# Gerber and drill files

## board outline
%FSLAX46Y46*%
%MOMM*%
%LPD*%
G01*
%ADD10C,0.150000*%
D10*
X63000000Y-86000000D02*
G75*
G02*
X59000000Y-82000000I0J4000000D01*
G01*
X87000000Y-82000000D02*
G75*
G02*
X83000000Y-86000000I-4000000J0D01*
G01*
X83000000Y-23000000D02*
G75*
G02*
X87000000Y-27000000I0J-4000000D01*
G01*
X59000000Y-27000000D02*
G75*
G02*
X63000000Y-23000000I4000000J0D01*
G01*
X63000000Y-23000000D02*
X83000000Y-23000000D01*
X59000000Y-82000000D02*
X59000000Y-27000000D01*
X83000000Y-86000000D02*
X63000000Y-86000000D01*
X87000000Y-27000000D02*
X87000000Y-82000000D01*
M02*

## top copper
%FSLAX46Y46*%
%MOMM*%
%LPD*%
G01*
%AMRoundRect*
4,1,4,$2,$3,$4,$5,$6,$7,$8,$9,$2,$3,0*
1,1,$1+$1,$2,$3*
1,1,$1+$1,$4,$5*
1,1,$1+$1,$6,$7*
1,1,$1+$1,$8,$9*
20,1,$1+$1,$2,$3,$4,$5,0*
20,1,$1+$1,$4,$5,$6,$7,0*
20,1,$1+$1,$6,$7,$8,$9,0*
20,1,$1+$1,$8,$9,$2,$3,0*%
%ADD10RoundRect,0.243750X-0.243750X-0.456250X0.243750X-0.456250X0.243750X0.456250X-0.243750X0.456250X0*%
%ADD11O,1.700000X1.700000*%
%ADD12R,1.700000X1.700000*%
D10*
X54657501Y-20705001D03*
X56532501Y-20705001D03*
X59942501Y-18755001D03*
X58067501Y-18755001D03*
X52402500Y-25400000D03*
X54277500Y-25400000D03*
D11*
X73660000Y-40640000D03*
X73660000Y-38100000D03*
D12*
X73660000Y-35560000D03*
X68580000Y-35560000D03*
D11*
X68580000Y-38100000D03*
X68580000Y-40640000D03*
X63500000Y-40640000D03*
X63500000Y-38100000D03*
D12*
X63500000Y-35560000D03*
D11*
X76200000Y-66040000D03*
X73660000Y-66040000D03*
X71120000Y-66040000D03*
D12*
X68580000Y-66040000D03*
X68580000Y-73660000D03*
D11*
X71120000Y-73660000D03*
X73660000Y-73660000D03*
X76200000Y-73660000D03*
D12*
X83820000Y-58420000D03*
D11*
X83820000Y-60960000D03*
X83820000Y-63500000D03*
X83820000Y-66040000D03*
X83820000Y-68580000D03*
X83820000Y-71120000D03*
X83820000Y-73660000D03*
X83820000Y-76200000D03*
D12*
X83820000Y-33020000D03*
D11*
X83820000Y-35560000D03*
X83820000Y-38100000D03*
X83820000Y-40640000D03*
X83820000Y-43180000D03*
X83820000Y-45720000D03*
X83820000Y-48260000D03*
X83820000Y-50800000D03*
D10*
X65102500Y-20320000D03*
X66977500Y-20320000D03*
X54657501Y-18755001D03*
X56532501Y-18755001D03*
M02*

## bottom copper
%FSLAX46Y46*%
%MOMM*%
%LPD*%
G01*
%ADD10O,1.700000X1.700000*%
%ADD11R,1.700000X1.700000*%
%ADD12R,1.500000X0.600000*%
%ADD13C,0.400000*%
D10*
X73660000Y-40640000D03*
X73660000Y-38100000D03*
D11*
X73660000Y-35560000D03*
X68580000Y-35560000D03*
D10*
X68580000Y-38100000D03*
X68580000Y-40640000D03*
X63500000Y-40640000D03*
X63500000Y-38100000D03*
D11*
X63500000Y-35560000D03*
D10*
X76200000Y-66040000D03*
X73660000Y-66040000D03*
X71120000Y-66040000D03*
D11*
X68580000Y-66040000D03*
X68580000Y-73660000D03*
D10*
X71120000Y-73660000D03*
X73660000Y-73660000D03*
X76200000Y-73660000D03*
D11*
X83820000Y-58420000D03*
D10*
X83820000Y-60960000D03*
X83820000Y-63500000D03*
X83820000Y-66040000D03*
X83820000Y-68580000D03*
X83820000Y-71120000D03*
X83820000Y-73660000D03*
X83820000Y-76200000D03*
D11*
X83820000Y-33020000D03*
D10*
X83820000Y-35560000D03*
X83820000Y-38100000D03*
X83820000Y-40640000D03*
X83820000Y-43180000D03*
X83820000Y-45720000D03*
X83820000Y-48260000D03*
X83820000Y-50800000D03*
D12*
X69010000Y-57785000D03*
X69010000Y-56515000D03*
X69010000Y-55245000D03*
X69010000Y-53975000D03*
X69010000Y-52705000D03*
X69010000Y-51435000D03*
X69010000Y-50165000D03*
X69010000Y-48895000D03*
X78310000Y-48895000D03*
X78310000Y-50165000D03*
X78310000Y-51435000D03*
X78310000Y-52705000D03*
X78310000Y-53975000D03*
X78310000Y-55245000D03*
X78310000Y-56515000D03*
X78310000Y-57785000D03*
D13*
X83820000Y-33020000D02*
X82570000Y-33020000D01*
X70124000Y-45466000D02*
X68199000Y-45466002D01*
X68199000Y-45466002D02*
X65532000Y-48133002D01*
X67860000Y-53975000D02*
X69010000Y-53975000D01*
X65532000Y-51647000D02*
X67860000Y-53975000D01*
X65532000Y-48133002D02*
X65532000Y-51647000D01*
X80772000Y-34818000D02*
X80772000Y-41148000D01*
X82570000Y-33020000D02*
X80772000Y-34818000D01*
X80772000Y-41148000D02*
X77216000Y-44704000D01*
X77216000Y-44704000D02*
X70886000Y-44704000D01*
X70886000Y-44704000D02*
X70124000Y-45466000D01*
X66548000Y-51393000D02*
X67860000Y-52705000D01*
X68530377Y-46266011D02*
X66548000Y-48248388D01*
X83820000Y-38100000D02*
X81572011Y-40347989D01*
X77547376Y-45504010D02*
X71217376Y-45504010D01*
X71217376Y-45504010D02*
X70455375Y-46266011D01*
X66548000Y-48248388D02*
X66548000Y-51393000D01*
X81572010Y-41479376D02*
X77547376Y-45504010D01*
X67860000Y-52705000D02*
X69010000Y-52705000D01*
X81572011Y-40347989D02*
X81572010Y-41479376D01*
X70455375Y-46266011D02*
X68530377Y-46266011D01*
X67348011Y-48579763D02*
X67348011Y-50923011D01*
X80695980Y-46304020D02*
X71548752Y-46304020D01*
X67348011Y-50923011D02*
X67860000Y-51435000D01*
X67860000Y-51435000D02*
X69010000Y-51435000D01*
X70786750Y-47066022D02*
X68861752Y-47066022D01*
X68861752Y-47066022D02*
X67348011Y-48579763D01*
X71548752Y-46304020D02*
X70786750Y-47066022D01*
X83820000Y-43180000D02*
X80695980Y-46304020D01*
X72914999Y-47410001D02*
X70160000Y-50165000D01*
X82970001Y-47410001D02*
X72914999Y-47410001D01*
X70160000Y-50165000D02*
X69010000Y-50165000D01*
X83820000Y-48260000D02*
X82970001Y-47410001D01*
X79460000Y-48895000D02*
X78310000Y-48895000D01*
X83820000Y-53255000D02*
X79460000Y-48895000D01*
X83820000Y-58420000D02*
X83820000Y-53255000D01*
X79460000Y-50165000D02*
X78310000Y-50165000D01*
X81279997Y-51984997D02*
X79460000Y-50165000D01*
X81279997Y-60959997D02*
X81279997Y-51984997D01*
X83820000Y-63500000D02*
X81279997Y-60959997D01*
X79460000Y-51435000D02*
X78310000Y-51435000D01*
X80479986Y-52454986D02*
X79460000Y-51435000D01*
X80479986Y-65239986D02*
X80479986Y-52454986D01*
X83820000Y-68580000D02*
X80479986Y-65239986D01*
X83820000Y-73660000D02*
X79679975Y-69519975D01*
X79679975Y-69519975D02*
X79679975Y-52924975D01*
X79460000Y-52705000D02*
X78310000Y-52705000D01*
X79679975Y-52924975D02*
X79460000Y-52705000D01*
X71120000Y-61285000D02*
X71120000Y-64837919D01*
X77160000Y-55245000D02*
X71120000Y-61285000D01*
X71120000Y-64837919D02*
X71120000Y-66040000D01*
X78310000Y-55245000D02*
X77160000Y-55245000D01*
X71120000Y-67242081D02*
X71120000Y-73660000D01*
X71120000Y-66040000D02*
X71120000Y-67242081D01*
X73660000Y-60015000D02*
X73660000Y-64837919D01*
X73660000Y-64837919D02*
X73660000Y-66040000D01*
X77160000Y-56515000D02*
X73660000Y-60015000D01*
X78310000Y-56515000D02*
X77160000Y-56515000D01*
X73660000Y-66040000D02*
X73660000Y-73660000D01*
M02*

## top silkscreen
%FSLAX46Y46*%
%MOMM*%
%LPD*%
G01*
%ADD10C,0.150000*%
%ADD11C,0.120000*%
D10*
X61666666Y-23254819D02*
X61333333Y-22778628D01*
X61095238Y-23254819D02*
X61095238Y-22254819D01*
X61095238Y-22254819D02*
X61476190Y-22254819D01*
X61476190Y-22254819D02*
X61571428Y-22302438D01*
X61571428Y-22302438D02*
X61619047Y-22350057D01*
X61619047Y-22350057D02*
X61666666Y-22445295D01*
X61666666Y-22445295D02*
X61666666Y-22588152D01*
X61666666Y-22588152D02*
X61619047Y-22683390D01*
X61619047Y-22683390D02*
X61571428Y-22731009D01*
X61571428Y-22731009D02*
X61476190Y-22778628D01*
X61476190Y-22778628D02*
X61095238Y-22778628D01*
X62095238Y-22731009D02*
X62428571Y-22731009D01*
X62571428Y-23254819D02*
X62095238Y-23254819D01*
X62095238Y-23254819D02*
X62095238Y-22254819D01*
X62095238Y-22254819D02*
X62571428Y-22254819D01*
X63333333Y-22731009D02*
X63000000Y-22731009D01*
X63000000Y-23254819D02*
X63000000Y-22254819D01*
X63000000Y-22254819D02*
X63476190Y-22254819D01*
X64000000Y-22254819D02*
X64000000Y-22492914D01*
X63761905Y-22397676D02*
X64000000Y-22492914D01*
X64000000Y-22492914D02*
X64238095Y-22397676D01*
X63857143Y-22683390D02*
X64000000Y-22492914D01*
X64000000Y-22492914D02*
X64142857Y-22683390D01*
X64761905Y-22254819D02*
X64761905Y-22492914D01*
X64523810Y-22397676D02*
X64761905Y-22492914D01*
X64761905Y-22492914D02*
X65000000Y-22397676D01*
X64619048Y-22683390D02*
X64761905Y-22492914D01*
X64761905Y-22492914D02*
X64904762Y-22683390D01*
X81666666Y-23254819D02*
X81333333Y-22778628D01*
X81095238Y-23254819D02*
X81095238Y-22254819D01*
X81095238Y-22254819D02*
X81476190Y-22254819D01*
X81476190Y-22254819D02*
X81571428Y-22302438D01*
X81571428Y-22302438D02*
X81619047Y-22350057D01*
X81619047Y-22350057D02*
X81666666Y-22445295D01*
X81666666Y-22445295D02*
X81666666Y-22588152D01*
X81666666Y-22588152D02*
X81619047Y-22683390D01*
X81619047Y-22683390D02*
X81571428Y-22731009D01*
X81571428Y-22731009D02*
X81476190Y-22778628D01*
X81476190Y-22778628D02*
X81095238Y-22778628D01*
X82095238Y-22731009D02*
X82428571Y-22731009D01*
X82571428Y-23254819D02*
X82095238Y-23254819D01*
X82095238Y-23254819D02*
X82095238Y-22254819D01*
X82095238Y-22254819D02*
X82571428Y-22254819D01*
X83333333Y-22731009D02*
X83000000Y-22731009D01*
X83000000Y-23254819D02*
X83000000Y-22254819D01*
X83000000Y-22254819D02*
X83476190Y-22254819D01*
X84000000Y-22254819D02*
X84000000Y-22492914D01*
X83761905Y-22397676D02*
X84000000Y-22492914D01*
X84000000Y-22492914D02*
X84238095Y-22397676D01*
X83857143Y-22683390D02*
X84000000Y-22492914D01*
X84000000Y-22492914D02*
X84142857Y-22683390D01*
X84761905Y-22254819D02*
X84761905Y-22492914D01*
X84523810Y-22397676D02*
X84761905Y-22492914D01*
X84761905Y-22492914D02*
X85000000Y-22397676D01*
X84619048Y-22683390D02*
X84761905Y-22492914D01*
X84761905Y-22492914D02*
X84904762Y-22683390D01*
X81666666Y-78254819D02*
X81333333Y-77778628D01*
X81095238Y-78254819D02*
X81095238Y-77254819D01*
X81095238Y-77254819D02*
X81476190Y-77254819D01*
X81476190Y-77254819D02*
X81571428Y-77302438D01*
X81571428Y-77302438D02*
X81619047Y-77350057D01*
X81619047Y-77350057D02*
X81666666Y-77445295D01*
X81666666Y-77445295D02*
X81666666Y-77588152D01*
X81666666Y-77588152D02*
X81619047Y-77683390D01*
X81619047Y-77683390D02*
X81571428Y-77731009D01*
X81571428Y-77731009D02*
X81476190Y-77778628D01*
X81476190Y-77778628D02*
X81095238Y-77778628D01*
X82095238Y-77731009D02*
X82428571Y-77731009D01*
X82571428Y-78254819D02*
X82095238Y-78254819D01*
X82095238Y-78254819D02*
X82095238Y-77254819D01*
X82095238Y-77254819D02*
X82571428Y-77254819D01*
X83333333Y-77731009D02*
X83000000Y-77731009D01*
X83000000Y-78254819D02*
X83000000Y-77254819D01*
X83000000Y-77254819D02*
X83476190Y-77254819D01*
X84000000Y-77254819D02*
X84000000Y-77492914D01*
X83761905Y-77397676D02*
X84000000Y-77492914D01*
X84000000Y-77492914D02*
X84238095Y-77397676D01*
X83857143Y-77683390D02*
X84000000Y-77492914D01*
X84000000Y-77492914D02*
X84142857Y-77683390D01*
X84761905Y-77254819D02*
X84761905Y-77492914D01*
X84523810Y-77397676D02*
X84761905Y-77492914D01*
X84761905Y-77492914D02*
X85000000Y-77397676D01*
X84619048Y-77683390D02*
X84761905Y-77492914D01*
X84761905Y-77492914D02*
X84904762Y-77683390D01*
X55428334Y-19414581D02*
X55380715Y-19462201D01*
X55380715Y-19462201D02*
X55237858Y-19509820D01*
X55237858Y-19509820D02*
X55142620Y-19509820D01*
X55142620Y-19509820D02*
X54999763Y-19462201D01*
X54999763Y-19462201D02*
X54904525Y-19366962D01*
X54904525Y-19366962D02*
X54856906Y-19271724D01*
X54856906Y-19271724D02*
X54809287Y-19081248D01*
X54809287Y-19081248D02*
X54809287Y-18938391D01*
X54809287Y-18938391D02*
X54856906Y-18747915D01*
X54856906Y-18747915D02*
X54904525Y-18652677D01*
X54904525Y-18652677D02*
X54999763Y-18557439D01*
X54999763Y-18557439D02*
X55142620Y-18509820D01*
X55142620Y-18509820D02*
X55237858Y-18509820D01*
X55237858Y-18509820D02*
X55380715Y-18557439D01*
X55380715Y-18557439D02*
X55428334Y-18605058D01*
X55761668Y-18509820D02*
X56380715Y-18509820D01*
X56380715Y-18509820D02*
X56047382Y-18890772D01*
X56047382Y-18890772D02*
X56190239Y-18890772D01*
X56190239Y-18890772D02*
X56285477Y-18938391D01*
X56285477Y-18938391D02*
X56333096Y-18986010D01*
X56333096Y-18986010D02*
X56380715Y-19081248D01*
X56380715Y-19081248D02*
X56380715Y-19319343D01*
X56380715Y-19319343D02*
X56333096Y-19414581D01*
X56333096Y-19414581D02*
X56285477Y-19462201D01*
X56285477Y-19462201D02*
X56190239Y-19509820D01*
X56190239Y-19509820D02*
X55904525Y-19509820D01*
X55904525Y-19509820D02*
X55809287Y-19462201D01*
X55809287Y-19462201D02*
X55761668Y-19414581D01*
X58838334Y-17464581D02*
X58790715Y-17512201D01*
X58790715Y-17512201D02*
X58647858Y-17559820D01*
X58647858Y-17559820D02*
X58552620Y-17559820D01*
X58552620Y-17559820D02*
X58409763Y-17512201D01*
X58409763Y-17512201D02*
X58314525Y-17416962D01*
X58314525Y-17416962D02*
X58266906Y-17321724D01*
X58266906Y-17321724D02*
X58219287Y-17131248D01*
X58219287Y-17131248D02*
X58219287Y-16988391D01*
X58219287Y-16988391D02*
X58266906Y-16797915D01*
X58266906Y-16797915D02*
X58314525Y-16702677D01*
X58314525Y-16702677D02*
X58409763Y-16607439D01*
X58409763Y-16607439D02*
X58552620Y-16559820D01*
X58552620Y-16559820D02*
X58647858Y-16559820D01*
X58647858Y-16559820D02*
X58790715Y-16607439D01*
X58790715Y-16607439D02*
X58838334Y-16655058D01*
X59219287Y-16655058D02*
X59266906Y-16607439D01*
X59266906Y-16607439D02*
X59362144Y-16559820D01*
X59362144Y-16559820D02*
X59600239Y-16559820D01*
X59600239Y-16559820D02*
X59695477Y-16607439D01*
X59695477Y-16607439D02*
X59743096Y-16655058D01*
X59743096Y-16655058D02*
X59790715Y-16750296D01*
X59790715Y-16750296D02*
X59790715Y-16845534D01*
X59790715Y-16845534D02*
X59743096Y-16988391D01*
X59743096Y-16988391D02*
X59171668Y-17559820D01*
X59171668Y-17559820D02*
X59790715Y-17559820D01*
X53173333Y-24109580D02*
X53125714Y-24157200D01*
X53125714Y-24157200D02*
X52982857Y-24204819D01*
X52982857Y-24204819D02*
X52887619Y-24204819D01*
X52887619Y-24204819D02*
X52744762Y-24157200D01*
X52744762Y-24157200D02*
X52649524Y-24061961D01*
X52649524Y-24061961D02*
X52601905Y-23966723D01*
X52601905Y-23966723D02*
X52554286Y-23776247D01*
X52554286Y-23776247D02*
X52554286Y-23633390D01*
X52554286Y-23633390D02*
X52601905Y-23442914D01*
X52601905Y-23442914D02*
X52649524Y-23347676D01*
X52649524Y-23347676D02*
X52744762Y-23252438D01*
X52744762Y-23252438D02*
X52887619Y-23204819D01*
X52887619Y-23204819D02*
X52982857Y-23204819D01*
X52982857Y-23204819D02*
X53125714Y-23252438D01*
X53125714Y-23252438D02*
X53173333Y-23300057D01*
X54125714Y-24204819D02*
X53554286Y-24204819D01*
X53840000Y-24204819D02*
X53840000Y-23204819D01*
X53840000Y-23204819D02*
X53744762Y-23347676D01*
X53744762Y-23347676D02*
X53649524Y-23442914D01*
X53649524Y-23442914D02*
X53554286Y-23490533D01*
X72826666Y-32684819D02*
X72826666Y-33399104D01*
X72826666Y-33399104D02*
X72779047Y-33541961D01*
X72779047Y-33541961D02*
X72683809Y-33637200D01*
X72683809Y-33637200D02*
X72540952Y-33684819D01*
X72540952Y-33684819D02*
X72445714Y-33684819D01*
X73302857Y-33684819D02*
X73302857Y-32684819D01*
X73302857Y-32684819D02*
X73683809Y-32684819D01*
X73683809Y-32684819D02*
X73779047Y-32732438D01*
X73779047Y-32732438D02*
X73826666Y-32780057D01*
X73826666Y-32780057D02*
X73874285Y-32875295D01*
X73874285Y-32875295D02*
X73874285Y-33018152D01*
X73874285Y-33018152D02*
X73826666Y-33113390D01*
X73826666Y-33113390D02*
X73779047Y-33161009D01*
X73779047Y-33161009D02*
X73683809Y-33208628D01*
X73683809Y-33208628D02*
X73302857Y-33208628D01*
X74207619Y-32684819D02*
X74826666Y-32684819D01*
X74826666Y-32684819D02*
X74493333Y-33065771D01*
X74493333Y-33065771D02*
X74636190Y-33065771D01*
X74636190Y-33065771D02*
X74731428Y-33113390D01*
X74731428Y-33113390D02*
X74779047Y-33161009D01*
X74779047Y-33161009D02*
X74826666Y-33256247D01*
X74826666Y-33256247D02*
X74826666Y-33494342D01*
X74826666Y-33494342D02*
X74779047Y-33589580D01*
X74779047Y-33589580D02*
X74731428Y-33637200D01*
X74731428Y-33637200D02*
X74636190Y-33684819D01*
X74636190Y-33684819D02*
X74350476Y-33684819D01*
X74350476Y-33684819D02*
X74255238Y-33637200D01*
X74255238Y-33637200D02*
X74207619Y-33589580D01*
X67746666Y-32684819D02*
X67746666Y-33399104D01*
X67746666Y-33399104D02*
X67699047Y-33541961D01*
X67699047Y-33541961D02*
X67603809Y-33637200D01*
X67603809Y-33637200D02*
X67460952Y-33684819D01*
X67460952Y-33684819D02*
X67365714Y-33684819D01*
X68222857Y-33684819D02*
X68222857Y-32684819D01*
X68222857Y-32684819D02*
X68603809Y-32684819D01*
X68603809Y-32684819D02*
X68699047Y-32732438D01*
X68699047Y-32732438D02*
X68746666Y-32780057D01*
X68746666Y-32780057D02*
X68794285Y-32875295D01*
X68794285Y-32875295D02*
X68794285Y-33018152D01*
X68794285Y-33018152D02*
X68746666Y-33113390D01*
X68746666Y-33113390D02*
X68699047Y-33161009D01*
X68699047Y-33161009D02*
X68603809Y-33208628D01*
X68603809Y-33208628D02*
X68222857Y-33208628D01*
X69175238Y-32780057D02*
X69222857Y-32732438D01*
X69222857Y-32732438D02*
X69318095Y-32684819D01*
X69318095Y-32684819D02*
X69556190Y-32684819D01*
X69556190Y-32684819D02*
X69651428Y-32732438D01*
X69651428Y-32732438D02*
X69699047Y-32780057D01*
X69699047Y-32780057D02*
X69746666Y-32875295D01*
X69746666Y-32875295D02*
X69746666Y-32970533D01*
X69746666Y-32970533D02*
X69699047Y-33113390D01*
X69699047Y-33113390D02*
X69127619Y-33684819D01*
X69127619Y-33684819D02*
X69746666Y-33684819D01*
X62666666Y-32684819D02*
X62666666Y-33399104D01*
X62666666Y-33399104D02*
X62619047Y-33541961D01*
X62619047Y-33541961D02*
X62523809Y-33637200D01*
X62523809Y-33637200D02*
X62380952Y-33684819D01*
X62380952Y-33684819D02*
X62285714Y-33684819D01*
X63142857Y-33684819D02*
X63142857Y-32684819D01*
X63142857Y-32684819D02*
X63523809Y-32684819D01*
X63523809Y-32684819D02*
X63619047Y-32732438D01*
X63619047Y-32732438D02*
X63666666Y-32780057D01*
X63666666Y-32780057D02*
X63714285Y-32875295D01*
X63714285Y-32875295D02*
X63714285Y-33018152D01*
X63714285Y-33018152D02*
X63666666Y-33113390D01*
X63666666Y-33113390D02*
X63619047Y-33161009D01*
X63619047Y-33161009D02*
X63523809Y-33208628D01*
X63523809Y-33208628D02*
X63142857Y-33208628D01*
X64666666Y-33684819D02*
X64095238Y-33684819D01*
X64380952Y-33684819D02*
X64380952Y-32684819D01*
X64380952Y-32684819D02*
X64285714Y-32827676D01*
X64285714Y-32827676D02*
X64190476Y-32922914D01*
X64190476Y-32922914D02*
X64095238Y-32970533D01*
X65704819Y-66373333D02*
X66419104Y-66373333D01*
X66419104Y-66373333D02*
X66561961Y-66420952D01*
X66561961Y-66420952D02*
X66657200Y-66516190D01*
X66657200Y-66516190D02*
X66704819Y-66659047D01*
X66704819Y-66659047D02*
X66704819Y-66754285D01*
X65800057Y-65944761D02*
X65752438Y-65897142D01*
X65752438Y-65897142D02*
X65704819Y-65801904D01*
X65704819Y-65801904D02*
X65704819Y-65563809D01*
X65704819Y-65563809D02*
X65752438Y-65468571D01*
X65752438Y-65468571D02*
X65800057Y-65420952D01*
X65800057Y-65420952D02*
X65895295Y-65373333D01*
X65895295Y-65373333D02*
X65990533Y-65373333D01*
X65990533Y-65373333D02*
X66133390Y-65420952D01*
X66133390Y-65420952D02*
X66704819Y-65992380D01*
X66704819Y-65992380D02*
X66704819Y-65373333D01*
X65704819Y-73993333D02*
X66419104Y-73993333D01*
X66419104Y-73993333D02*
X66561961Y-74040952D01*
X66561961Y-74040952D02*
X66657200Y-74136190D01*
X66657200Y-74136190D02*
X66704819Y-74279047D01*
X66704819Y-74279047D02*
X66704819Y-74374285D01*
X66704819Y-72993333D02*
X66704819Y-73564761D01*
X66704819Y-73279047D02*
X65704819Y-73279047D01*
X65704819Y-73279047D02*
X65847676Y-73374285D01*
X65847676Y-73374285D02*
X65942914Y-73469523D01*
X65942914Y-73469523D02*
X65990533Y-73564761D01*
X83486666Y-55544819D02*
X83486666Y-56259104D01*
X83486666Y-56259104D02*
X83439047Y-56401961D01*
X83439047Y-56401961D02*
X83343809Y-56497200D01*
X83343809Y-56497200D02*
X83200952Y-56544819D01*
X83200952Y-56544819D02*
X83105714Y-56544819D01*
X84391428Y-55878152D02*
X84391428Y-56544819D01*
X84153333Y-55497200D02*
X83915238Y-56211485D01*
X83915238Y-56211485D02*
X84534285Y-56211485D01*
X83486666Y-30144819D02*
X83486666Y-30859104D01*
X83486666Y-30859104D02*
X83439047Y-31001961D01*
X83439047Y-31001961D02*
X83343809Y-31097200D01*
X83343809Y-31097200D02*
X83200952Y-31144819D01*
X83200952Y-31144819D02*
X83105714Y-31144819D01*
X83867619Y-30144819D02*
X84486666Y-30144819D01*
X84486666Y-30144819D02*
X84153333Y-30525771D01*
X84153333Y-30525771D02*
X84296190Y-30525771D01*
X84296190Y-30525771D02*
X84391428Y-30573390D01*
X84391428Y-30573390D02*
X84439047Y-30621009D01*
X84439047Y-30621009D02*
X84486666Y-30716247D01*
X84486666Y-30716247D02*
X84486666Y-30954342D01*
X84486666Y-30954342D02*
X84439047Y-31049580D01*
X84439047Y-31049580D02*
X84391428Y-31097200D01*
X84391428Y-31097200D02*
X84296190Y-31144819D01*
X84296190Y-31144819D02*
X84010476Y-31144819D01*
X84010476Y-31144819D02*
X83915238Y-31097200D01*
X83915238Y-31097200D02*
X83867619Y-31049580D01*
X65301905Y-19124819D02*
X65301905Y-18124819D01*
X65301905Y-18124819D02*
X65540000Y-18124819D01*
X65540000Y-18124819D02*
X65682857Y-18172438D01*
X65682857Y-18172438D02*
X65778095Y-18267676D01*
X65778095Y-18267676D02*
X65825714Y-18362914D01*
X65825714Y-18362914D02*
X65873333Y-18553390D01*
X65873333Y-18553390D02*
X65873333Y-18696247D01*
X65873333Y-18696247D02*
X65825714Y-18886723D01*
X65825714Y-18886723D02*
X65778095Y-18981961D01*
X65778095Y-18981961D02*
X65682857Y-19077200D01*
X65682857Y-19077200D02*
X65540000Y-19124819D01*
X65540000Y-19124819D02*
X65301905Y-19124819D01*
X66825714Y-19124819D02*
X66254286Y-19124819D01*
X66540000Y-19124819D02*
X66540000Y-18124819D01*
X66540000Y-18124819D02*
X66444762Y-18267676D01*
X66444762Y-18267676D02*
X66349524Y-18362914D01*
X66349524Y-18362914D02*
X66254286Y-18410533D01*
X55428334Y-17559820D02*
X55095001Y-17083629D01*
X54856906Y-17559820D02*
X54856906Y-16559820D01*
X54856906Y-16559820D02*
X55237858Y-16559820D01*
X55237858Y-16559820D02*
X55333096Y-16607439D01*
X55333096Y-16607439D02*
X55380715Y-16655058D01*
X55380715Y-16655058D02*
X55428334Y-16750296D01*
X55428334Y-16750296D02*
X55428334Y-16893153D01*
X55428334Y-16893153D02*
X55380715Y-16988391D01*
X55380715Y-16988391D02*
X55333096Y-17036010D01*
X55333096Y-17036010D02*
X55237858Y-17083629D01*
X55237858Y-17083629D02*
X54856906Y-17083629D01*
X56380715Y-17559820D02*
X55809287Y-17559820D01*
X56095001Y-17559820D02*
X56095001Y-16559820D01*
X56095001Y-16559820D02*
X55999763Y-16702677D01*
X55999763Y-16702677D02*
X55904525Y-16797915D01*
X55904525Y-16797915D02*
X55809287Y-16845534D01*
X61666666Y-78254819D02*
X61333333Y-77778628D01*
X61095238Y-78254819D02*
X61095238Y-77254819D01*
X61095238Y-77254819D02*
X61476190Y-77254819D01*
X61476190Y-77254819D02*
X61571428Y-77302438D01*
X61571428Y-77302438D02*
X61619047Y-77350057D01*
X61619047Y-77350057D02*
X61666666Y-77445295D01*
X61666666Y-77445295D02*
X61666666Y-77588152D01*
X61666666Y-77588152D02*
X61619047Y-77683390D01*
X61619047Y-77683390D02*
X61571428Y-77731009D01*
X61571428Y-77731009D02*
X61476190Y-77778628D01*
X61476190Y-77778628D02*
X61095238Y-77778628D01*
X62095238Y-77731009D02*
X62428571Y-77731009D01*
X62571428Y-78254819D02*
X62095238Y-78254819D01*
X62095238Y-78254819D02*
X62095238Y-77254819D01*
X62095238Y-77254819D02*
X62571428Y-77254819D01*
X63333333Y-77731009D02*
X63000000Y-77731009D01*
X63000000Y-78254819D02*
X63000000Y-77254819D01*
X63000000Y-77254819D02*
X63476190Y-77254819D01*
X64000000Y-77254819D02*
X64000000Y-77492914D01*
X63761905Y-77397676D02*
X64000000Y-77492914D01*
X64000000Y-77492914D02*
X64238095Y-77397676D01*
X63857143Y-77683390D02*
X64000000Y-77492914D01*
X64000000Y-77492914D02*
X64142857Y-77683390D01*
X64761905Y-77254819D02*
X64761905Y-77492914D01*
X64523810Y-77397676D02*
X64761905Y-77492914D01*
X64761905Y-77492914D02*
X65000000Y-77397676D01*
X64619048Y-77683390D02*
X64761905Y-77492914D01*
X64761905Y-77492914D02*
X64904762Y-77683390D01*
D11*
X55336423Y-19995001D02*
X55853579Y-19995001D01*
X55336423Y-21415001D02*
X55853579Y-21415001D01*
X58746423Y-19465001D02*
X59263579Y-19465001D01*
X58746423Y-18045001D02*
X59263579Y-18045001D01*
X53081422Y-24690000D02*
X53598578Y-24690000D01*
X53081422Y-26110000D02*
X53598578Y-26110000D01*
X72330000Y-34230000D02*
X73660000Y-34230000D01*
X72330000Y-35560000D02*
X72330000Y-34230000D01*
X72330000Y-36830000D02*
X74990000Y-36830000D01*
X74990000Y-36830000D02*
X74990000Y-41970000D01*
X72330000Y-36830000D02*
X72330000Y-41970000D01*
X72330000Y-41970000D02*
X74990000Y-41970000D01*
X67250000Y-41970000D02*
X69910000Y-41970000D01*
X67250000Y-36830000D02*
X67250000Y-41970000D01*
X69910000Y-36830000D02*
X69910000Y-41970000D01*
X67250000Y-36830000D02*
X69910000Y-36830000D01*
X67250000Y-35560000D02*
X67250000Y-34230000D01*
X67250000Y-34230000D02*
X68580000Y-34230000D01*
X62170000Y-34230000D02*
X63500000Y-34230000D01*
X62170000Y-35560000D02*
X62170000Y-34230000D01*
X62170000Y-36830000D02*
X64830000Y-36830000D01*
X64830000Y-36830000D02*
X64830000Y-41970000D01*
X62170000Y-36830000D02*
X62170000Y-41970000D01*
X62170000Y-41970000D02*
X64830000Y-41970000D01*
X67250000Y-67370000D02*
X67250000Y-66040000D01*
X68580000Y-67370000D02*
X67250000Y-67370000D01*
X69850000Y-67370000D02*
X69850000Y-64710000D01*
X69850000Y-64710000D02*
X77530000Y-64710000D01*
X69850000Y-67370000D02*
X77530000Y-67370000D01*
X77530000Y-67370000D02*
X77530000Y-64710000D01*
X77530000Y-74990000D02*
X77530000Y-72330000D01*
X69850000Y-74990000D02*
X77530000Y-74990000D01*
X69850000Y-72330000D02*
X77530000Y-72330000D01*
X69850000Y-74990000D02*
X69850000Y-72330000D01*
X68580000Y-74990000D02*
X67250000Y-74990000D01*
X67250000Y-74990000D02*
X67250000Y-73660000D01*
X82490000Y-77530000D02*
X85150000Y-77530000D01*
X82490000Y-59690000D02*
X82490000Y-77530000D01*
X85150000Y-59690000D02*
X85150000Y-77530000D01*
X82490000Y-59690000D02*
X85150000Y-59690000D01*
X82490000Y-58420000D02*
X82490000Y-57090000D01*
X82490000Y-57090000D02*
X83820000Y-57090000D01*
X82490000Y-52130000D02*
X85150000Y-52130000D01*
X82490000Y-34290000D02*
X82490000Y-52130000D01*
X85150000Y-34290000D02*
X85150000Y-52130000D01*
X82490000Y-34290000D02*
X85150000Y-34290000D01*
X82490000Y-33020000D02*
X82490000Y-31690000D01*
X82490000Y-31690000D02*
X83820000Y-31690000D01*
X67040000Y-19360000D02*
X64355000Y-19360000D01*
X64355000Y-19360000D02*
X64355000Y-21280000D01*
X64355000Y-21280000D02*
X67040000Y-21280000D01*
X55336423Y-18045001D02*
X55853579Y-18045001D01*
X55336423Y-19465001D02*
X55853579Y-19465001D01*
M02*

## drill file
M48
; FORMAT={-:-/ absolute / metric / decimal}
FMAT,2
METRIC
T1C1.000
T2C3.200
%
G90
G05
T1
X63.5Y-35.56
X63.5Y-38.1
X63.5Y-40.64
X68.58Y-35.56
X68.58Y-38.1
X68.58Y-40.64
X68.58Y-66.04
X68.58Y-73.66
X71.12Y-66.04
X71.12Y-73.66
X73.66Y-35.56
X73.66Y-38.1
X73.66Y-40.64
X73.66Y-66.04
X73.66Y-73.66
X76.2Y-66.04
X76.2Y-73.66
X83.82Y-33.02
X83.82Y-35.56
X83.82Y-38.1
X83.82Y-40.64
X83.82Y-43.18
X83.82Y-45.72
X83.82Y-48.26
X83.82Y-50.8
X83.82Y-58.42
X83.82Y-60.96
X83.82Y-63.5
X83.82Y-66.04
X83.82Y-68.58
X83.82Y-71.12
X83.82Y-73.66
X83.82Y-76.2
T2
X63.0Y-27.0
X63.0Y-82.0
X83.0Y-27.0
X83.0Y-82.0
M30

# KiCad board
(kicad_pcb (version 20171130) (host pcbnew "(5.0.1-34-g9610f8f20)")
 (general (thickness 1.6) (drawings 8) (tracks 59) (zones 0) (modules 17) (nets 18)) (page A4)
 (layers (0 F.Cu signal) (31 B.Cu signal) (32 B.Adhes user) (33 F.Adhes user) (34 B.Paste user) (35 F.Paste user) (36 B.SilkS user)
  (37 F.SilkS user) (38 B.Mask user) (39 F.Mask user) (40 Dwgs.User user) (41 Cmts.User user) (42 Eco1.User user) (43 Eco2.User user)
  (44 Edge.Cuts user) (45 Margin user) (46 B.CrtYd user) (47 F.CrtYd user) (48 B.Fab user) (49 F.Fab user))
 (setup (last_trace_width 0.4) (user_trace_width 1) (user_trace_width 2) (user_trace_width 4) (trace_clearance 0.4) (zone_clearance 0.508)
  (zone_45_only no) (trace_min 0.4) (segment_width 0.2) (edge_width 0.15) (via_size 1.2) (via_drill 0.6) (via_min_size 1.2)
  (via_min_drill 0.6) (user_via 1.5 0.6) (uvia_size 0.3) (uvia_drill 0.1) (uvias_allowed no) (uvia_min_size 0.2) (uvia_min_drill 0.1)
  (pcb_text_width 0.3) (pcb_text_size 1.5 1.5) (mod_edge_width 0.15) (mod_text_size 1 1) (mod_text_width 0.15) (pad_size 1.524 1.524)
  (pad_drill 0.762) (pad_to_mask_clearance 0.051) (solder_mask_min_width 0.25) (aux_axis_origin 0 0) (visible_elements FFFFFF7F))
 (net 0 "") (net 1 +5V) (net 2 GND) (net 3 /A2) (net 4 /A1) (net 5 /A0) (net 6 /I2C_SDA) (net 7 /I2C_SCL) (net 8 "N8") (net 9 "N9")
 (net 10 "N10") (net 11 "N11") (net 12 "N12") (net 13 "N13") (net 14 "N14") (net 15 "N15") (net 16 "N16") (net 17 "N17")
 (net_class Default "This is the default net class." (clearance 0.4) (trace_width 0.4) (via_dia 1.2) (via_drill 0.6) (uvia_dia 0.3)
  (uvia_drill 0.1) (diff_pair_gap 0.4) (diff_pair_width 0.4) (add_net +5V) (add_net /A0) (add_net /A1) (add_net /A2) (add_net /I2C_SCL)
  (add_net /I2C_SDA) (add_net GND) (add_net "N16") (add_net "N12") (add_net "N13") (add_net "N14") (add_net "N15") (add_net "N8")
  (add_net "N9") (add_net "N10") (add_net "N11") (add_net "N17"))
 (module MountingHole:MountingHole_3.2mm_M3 (layer F.Cu) (at 63 27)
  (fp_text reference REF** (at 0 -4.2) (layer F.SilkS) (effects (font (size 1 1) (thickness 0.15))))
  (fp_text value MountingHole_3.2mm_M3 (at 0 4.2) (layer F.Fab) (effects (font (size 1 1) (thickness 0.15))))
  (pad 1 np_thru_hole circle (at 0 0) (size 3.2 3.2) (drill 3.2) (layers *.Cu *.Mask)))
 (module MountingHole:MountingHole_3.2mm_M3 (layer F.Cu) (at 83 27)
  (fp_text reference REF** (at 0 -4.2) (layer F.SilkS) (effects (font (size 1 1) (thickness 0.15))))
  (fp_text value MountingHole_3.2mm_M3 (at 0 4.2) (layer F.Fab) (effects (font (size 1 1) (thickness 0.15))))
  (pad 1 np_thru_hole circle (at 0 0) (size 3.2 3.2) (drill 3.2) (layers *.Cu *.Mask)))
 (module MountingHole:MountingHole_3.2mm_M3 (layer F.Cu) (at 83 82)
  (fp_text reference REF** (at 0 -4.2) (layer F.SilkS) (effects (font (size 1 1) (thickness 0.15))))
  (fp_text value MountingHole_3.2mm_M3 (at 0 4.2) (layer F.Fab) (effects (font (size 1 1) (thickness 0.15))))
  (pad 1 np_thru_hole circle (at 0 0) (size 3.2 3.2) (drill 3.2) (layers *.Cu *.Mask)))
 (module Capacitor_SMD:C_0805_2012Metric (layer F.Cu) (at 55.595001 20.705001)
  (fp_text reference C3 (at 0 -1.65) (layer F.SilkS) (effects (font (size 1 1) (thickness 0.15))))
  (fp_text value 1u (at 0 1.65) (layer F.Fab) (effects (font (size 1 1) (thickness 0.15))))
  (fp_line (start -0.258578 -0.71) (end 0.258578 -0.71) (layer F.SilkS) (width 0.12))
  (fp_line (start -0.258578 0.71) (end 0.258578 0.71) (layer F.SilkS) (width 0.12))
  (pad 1 smd roundrect (at -0.9375 0) (size 0.975 1.4) (layers F.Cu F.Paste F.Mask) (roundrect_rratio 0.25) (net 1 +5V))
  (pad 2 smd roundrect (at 0.9375 0) (size 0.975 1.4) (layers F.Cu F.Paste F.Mask) (roundrect_rratio 0.25) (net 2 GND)))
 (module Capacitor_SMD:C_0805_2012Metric (layer F.Cu) (at 59.005001 18.755001)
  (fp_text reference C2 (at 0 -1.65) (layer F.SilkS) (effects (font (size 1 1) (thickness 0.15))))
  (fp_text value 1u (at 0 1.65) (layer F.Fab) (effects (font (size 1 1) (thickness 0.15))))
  (fp_line (start -0.258578 0.71) (end 0.258578 0.71) (layer F.SilkS) (width 0.12))
  (fp_line (start -0.258578 -0.71) (end 0.258578 -0.71) (layer F.SilkS) (width 0.12))
  (pad 2 smd roundrect (at 0.9375 0) (size 0.975 1.4) (layers F.Cu F.Paste F.Mask) (roundrect_rratio 0.25) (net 2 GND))
  (pad 1 smd roundrect (at -0.9375 0) (size 0.975 1.4) (layers F.Cu F.Paste F.Mask) (roundrect_rratio 0.25) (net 1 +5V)))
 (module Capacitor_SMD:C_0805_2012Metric (layer F.Cu) (at 53.34 25.4)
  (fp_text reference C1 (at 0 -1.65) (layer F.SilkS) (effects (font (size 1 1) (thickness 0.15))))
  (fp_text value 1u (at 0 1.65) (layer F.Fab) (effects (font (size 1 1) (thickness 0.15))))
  (fp_line (start -0.258578 -0.71) (end 0.258578 -0.71) (layer F.SilkS) (width 0.12))
  (fp_line (start -0.258578 0.71) (end 0.258578 0.71) (layer F.SilkS) (width 0.12))
  (pad 1 smd roundrect (at -0.9375 0) (size 0.975 1.4) (layers F.Cu F.Paste F.Mask) (roundrect_rratio 0.25) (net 1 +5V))
  (pad 2 smd roundrect (at 0.9375 0) (size 0.975 1.4) (layers F.Cu F.Paste F.Mask) (roundrect_rratio 0.25) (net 2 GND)))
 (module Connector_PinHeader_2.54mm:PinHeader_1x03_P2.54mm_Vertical (layer F.Cu) (at 73.66 35.56)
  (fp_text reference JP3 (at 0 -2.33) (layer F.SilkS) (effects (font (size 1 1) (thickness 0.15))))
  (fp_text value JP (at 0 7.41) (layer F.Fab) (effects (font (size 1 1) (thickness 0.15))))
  (fp_line (start -1.33 -1.33) (end 0 -1.33) (layer F.SilkS) (width 0.12))
  (fp_line (start -1.33 0) (end -1.33 -1.33) (layer F.SilkS) (width 0.12))
  (fp_line (start -1.33 1.27) (end 1.33 1.27) (layer F.SilkS) (width 0.12))
  (fp_line (start 1.33 1.27) (end 1.33 6.41) (layer F.SilkS) (width 0.12))
  (fp_line (start -1.33 1.27) (end -1.33 6.41) (layer F.SilkS) (width 0.12))
  (fp_line (start -1.33 6.41) (end 1.33 6.41) (layer F.SilkS) (width 0.12))
  (pad 3 thru_hole oval (at 0 5.08) (size 1.7 1.7) (drill 1) (layers *.Cu *.Mask) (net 1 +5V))
  (pad 2 thru_hole oval (at 0 2.54) (size 1.7 1.7) (drill 1) (layers *.Cu *.Mask) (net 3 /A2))
  (pad 1 thru_hole rect (at 0 0) (size 1.7 1.7) (drill 1) (layers *.Cu *.Mask) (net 2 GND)))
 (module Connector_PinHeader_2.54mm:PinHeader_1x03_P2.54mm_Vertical (layer F.Cu) (at 68.58 35.56)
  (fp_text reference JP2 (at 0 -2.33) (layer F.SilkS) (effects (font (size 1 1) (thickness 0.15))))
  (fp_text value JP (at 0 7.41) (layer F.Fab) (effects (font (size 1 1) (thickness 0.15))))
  (fp_line (start -1.33 6.41) (end 1.33 6.41) (layer F.SilkS) (width 0.12))
  (fp_line (start -1.33 1.27) (end -1.33 6.41) (layer F.SilkS) (width 0.12))
  (fp_line (start 1.33 1.27) (end 1.33 6.41) (layer F.SilkS) (width 0.12))
  (fp_line (start -1.33 1.27) (end 1.33 1.27) (layer F.SilkS) (width 0.12))
  (fp_line (start -1.33 0) (end -1.33 -1.33) (layer F.SilkS) (width 0.12))
  (fp_line (start -1.33 -1.33) (end 0 -1.33) (layer F.SilkS) (width 0.12))
  (pad 1 thru_hole rect (at 0 0) (size 1.7 1.7) (drill 1) (layers *.Cu *.Mask) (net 2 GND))
  (pad 2 thru_hole oval (at 0 2.54) (size 1.7 1.7) (drill 1) (layers *.Cu *.Mask) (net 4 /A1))
  (pad 3 thru_hole oval (at 0 5.08) (size 1.7 1.7) (drill 1) (layers *.Cu *.Mask) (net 1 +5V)))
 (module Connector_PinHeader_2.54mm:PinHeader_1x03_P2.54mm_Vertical (layer F.Cu) (at 63.5 35.56)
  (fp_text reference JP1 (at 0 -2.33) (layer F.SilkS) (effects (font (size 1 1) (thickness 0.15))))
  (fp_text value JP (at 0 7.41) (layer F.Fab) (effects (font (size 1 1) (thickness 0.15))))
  (fp_line (start -1.33 -1.33) (end 0 -1.33) (layer F.SilkS) (width 0.12))
  (fp_line (start -1.33 0) (end -1.33 -1.33) (layer F.SilkS) (width 0.12))
  (fp_line (start -1.33 1.27) (end 1.33 1.27) (layer F.SilkS) (width 0.12))
  (fp_line (start 1.33 1.27) (end 1.33 6.41) (layer F.SilkS) (width 0.12))
  (fp_line (start -1.33 1.27) (end -1.33 6.41) (layer F.SilkS) (width 0.12))
  (fp_line (start -1.33 6.41) (end 1.33 6.41) (layer F.SilkS) (width 0.12))
  (pad 3 thru_hole oval (at 0 5.08) (size 1.7 1.7) (drill 1) (layers *.Cu *.Mask) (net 1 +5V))
  (pad 2 thru_hole oval (at 0 2.54) (size 1.7 1.7) (drill 1) (layers *.Cu *.Mask) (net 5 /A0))
  (pad 1 thru_hole rect (at 0 0) (size 1.7 1.7) (drill 1) (layers *.Cu *.Mask) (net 2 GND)))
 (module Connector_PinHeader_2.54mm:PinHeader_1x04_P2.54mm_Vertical (layer F.Cu) (at 68.58 66.04 90)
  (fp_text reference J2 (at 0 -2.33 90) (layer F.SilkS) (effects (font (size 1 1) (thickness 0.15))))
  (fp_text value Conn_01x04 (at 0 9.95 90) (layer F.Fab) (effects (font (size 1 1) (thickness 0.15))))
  (fp_line (start -1.33 -1.33) (end 0 -1.33) (layer F.SilkS) (width 0.12))
  (fp_line (start -1.33 0) (end -1.33 -1.33) (layer F.SilkS) (width 0.12))
  (fp_line (start -1.33 1.27) (end 1.33 1.27) (layer F.SilkS) (width 0.12))
  (fp_line (start 1.33 1.27) (end 1.33 8.95) (layer F.SilkS) (width 0.12))
  (fp_line (start -1.33 1.27) (end -1.33 8.95) (layer F.SilkS) (width 0.12))
  (fp_line (start -1.33 8.95) (end 1.33 8.95) (layer F.SilkS) (width 0.12))
  (pad 4 thru_hole oval (at 0 7.62 90) (size 1.7 1.7) (drill 1) (layers *.Cu *.Mask) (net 2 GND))
  (pad 3 thru_hole oval (at 0 5.08 90) (size 1.7 1.7) (drill 1) (layers *.Cu *.Mask) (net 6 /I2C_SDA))
  (pad 2 thru_hole oval (at 0 2.54 90) (size 1.7 1.7) (drill 1) (layers *.Cu *.Mask) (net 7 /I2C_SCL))
  (pad 1 thru_hole rect (at 0 0 90) (size 1.7 1.7) (drill 1) (layers *.Cu *.Mask) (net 1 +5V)))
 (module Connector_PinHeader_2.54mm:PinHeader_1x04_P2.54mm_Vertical (layer F.Cu) (at 68.58 73.66 90)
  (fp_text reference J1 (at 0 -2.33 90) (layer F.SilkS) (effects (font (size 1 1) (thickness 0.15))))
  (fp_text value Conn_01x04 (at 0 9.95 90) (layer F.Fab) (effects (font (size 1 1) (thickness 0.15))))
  (fp_line (start -1.33 8.95) (end 1.33 8.95) (layer F.SilkS) (width 0.12))
  (fp_line (start -1.33 1.27) (end -1.33 8.95) (layer F.SilkS) (width 0.12))
  (fp_line (start 1.33 1.27) (end 1.33 8.95) (layer F.SilkS) (width 0.12))
  (fp_line (start -1.33 1.27) (end 1.33 1.27) (layer F.SilkS) (width 0.12))
  (fp_line (start -1.33 0) (end -1.33 -1.33) (layer F.SilkS) (width 0.12))
  (fp_line (start -1.33 -1.33) (end 0 -1.33) (layer F.SilkS) (width 0.12))
  (pad 1 thru_hole rect (at 0 0 90) (size 1.7 1.7) (drill 1) (layers *.Cu *.Mask) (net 1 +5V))
  (pad 2 thru_hole oval (at 0 2.54 90) (size 1.7 1.7) (drill 1) (layers *.Cu *.Mask) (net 7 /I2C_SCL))
  (pad 3 thru_hole oval (at 0 5.08 90) (size 1.7 1.7) (drill 1) (layers *.Cu *.Mask) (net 6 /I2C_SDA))
  (pad 4 thru_hole oval (at 0 7.62 90) (size 1.7 1.7) (drill 1) (layers *.Cu *.Mask) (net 2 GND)))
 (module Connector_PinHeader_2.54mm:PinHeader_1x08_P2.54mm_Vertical (layer F.Cu) (at 83.82 58.42)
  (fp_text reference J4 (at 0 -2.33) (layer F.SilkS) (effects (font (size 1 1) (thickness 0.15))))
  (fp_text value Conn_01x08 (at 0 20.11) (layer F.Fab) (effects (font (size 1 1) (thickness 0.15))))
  (fp_line (start -1.33 19.11) (end 1.33 19.11) (layer F.SilkS) (width 0.12))
  (fp_line (start -1.33 1.27) (end -1.33 19.11) (layer F.SilkS) (width 0.12))
  (fp_line (start 1.33 1.27) (end 1.33 19.11) (layer F.SilkS) (width 0.12))
  (fp_line (start -1.33 1.27) (end 1.33 1.27) (layer F.SilkS) (width 0.12))
  (fp_line (start -1.33 0) (end -1.33 -1.33) (layer F.SilkS) (width 0.12))
  (fp_line (start -1.33 -1.33) (end 0 -1.33) (layer F.SilkS) (width 0.12))
  (pad 1 thru_hole rect (at 0 0) (size 1.7 1.7) (drill 1) (layers *.Cu *.Mask) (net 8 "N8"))
  (pad 2 thru_hole oval (at 0 2.54) (size 1.7 1.7) (drill 1) (layers *.Cu *.Mask) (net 2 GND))
  (pad 3 thru_hole oval (at 0 5.08) (size 1.7 1.7) (drill 1) (layers *.Cu *.Mask) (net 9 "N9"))
  (pad 4 thru_hole oval (at 0 7.62) (size 1.7 1.7) (drill 1) (layers *.Cu *.Mask) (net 2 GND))
  (pad 5 thru_hole oval (at 0 10.16) (size 1.7 1.7) (drill 1) (layers *.Cu *.Mask) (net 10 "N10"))
  (pad 6 thru_hole oval (at 0 12.7) (size 1.7 1.7) (drill 1) (layers *.Cu *.Mask) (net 2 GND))
  (pad 7 thru_hole oval (at 0 15.24) (size 1.7 1.7) (drill 1) (layers *.Cu *.Mask) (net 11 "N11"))
  (pad 8 thru_hole oval (at 0 17.78) (size 1.7 1.7) (drill 1) (layers *.Cu *.Mask) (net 2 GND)))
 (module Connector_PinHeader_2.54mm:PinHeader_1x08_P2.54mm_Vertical (layer F.Cu) (at 83.82 33.02)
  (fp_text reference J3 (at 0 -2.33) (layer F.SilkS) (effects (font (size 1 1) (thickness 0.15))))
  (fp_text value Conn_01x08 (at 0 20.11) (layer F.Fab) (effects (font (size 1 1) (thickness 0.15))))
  (fp_line (start -1.33 19.11) (end 1.33 19.11) (layer F.SilkS) (width 0.12))
  (fp_line (start -1.33 1.27) (end -1.33 19.11) (layer F.SilkS) (width 0.12))
  (fp_line (start 1.33 1.27) (end 1.33 19.11) (layer F.SilkS) (width 0.12))
  (fp_line (start -1.33 1.27) (end 1.33 1.27) (layer F.SilkS) (width 0.12))
  (fp_line (start -1.33 0) (end -1.33 -1.33) (layer F.SilkS) (width 0.12))
  (fp_line (start -1.33 -1.33) (end 0 -1.33) (layer F.SilkS) (width 0.12))
  (pad 1 thru_hole rect (at 0 0) (size 1.7 1.7) (drill 1) (layers *.Cu *.Mask) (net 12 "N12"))
  (pad 2 thru_hole oval (at 0 2.54) (size 1.7 1.7) (drill 1) (layers *.Cu *.Mask) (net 2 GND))
  (pad 3 thru_hole oval (at 0 5.08) (size 1.7 1.7) (drill 1) (layers *.Cu *.Mask) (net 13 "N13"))
  (pad 4 thru_hole oval (at 0 7.62) (size 1.7 1.7) (drill 1) (layers *.Cu *.Mask) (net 2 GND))
  (pad 5 thru_hole oval (at 0 10.16) (size 1.7 1.7) (drill 1) (layers *.Cu *.Mask) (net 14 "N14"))
  (pad 6 thru_hole oval (at 0 12.7) (size 1.7 1.7) (drill 1) (layers *.Cu *.Mask) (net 2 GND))
  (pad 7 thru_hole oval (at 0 15.24) (size 1.7 1.7) (drill 1) (layers *.Cu *.Mask) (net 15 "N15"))
  (pad 8 thru_hole oval (at 0 17.78) (size 1.7 1.7) (drill 1) (layers *.Cu *.Mask) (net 2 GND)))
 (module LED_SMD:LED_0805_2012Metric (layer F.Cu) (at 66.04 20.32)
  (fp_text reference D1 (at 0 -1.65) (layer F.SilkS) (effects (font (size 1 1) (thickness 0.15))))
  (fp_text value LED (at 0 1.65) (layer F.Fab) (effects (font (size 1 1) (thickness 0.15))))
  (fp_line (start 1 -0.96) (end -1.685 -0.96) (layer F.SilkS) (width 0.12))
  (fp_line (start -1.685 -0.96) (end -1.685 0.96) (layer F.SilkS) (width 0.12))
  (fp_line (start -1.685 0.96) (end 1 0.96) (layer F.SilkS) (width 0.12))
  (pad 1 smd roundrect (at -0.9375 0) (size 0.975 1.4) (layers F.Cu F.Paste F.Mask) (roundrect_rratio 0.25) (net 2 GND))
  (pad 2 smd roundrect (at 0.9375 0) (size 0.975 1.4) (layers F.Cu F.Paste F.Mask) (roundrect_rratio 0.25) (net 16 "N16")))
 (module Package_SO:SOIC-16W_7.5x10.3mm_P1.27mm (layer B.Cu) (at 73.66 53.34)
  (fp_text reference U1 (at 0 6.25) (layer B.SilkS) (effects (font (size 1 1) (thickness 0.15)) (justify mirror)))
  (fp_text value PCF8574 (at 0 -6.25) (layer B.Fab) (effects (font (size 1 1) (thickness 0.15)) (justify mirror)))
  (pad 1 smd rect (at -4.65 4.445) (size 1.5 0.6) (layers B.Cu B.Paste B.Mask) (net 5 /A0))
  (pad 2 smd rect (at -4.65 3.175) (size 1.5 0.6) (layers B.Cu B.Paste B.Mask) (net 4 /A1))
  (pad 3 smd rect (at -4.65 1.905) (size 1.5 0.6) (layers B.Cu B.Paste B.Mask) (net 3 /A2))
  (pad 4 smd rect (at -4.65 0.635) (size 1.5 0.6) (layers B.Cu B.Paste B.Mask) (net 12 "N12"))
  (pad 5 smd rect (at -4.65 -0.635) (size 1.5 0.6) (layers B.Cu B.Paste B.Mask) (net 13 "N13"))
  (pad 6 smd rect (at -4.65 -1.905) (size 1.5 0.6) (layers B.Cu B.Paste B.Mask) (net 14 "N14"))
  (pad 7 smd rect (at -4.65 -3.175) (size 1.5 0.6) (layers B.Cu B.Paste B.Mask) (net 15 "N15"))
  (pad 8 smd rect (at -4.65 -4.445) (size 1.5 0.6) (layers B.Cu B.Paste B.Mask) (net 2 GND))
  (pad 9 smd rect (at 4.65 -4.445) (size 1.5 0.6) (layers B.Cu B.Paste B.Mask) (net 8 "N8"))
  (pad 10 smd rect (at 4.65 -3.175) (size 1.5 0.6) (layers B.Cu B.Paste B.Mask) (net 9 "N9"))
  (pad 11 smd rect (at 4.65 -1.905) (size 1.5 0.6) (layers B.Cu B.Paste B.Mask) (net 10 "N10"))
  (pad 12 smd rect (at 4.65 -0.635) (size 1.5 0.6) (layers B.Cu B.Paste B.Mask) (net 11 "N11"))
  (pad 13 smd rect (at 4.65 0.635) (size 1.5 0.6) (layers B.Cu B.Paste B.Mask) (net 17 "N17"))
  (pad 14 smd rect (at 4.65 1.905) (size 1.5 0.6) (layers B.Cu B.Paste B.Mask) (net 7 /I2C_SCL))
  (pad 15 smd rect (at 4.65 3.175) (size 1.5 0.6) (layers B.Cu B.Paste B.Mask) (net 6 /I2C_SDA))
  (pad 16 smd rect (at 4.65 4.445) (size 1.5 0.6) (layers B.Cu B.Paste B.Mask) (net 1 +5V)))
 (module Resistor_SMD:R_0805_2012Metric (layer F.Cu) (at 55.595001 18.755001)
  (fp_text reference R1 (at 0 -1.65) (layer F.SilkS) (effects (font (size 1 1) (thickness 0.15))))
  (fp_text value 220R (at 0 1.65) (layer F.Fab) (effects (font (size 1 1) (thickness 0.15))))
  (fp_line (start -0.258578 -0.71) (end 0.258578 -0.71) (layer F.SilkS) (width 0.12))
  (fp_line (start -0.258578 0.71) (end 0.258578 0.71) (layer F.SilkS) (width 0.12))
  (pad 1 smd roundrect (at -0.9375 0) (size 0.975 1.4) (layers F.Cu F.Paste F.Mask) (roundrect_rratio 0.25) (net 1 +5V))
  (pad 2 smd roundrect (at 0.9375 0) (size 0.975 1.4) (layers F.Cu F.Paste F.Mask) (roundrect_rratio 0.25) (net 16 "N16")))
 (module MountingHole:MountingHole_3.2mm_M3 (layer F.Cu) (at 63 82)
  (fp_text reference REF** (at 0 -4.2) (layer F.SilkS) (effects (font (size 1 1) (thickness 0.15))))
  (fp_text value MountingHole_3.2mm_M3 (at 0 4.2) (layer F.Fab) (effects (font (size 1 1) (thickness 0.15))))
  (pad 1 np_thru_hole circle (at 0 0) (size 3.2 3.2) (drill 3.2) (layers *.Cu *.Mask)))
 (gr_arc (start 63 82) (end 59 82) (angle -90) (layer Edge.Cuts) (width 0.15))
 (gr_arc (start 83 82) (end 83 86) (angle -90) (layer Edge.Cuts) (width 0.15))
 (gr_arc (start 83 27) (end 87 27) (angle -90) (layer Edge.Cuts) (width 0.15))
 (gr_arc (start 63 27) (end 63 23) (angle -90) (layer Edge.Cuts) (width 0.15))
 (gr_line (start 63 23) (end 83 23) (layer Edge.Cuts) (width 0.15))
 (gr_line (start 59 82) (end 59 27) (layer Edge.Cuts) (width 0.15))
 (gr_line (start 83 86) (end 63 86) (layer Edge.Cuts) (width 0.15))
 (gr_line (start 87 27) (end 87 82) (layer Edge.Cuts) (width 0.15))
 (segment (start 83.82 33.02) (end 82.57 33.02) (width 0.4) (layer B.Cu) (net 12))
 (segment (start 70.124 45.466) (end 68.199 45.466002) (width 0.4) (layer B.Cu) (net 12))
 (segment (start 68.199 45.466002) (end 65.532 48.133002) (width 0.4) (layer B.Cu) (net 12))
 (segment (start 67.86 53.975) (end 69.01 53.975) (width 0.4) (layer B.Cu) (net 12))
 (segment (start 65.532 51.647) (end 67.86 53.975) (width 0.4) (layer B.Cu) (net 12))
 (segment (start 65.532 48.133002) (end 65.532 51.647) (width 0.4) (layer B.Cu) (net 12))
 (segment (start 80.772 34.818) (end 80.772 41.148) (width 0.4) (layer B.Cu) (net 12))
 (segment (start 82.57 33.02) (end 80.772 34.818) (width 0.4) (layer B.Cu) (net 12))
 (segment (start 80.772 41.148) (end 77.216 44.704) (width 0.4) (layer B.Cu) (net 12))
 (segment (start 77.216 44.704) (end 70.886 44.704) (width 0.4) (layer B.Cu) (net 12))
 (segment (start 70.886 44.704) (end 70.124 45.466) (width 0.4) (layer B.Cu) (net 12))
 (segment (start 66.548 51.393) (end 67.86 52.705) (width 0.4) (layer B.Cu) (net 13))
 (segment (start 68.530377 46.266011) (end 66.548 48.248388) (width 0.4) (layer B.Cu) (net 13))
 (segment (start 83.82 38.1) (end 81.572011 40.347989) (width 0.4) (layer B.Cu) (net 13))
 (segment (start 77.547376 45.50401) (end 71.217376 45.50401) (width 0.4) (layer B.Cu) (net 13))
 (segment (start 71.217376 45.50401) (end 70.455375 46.266011) (width 0.4) (layer B.Cu) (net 13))
 (segment (start 66.548 48.248388) (end 66.548 51.393) (width 0.4) (layer B.Cu) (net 13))
 (segment (start 81.57201 41.479376) (end 77.547376 45.50401) (width 0.4) (layer B.Cu) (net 13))
 (segment (start 67.86 52.705) (end 69.01 52.705) (width 0.4) (layer B.Cu) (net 13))
 (segment (start 81.572011 40.347989) (end 81.57201 41.479376) (width 0.4) (layer B.Cu) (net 13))
 (segment (start 70.455375 46.266011) (end 68.530377 46.266011) (width 0.4) (layer B.Cu) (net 13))
 (segment (start 67.348011 48.579763) (end 67.348011 50.923011) (width 0.4) (layer B.Cu) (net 14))
 (segment (start 80.69598 46.30402) (end 71.548752 46.30402) (width 0.4) (layer B.Cu) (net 14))
 (segment (start 67.348011 50.923011) (end 67.86 51.435) (width 0.4) (layer B.Cu) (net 14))
 (segment (start 67.86 51.435) (end 69.01 51.435) (width 0.4) (layer B.Cu) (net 14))
 (segment (start 70.78675 47.066022) (end 68.861752 47.066022) (width 0.4) (layer B.Cu) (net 14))
 (segment (start 68.861752 47.066022) (end 67.348011 48.579763) (width 0.4) (layer B.Cu) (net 14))
 (segment (start 71.548752 46.30402) (end 70.78675 47.066022) (width 0.4) (layer B.Cu) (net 14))
 (segment (start 83.82 43.18) (end 80.69598 46.30402) (width 0.4) (layer B.Cu) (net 14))
 (segment (start 72.914999 47.410001) (end 70.16 50.165) (width 0.4) (layer B.Cu) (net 15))
 (segment (start 82.970001 47.410001) (end 72.914999 47.410001) (width 0.4) (layer B.Cu) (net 15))
 (segment (start 70.16 50.165) (end 69.01 50.165) (width 0.4) (layer B.Cu) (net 15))
 (segment (start 83.82 48.26) (end 82.970001 47.410001) (width 0.4) (layer B.Cu) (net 15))
 (segment (start 79.46 48.895) (end 78.31 48.895) (width 0.4) (layer B.Cu) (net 8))
 (segment (start 83.82 53.255) (end 79.46 48.895) (width 0.4) (layer B.Cu) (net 8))
 (segment (start 83.82 58.42) (end 83.82 53.255) (width 0.4) (layer B.Cu) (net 8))
 (segment (start 79.46 50.165) (end 78.31 50.165) (width 0.4) (layer B.Cu) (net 9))
 (segment (start 81.279997 51.984997) (end 79.46 50.165) (width 0.4) (layer B.Cu) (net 9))
 (segment (start 81.279997 60.959997) (end 81.279997 51.984997) (width 0.4) (layer B.Cu) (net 9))
 (segment (start 83.82 63.5) (end 81.279997 60.959997) (width 0.4) (layer B.Cu) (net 9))
 (segment (start 79.46 51.435) (end 78.31 51.435) (width 0.4) (layer B.Cu) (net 10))
 (segment (start 80.479986 52.454986) (end 79.46 51.435) (width 0.4) (layer B.Cu) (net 10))
 (segment (start 80.479986 65.239986) (end 80.479986 52.454986) (width 0.4) (layer B.Cu) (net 10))
 (segment (start 83.82 68.58) (end 80.479986 65.239986) (width 0.4) (layer B.Cu) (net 10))
 (segment (start 83.82 73.66) (end 79.679975 69.519975) (width 0.4) (layer B.Cu) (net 11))
 (segment (start 79.679975 69.519975) (end 79.679975 52.924975) (width 0.4) (layer B.Cu) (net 11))
 (segment (start 79.46 52.705) (end 78.31 52.705) (width 0.4) (layer B.Cu) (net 11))
 (segment (start 79.679975 52.924975) (end 79.46 52.705) (width 0.4) (layer B.Cu) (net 11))
 (segment (start 71.12 61.285) (end 71.12 64.837919) (width 0.4) (layer B.Cu) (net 7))
 (segment (start 77.16 55.245) (end 71.12 61.285) (width 0.4) (layer B.Cu) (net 7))
 (segment (start 71.12 64.837919) (end 71.12 66.04) (width 0.4) (layer B.Cu) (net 7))
 (segment (start 78.31 55.245) (end 77.16 55.245) (width 0.4) (layer B.Cu) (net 7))
 (segment (start 71.12 67.242081) (end 71.12 73.66) (width 0.4) (layer B.Cu) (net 7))
 (segment (start 71.12 66.04) (end 71.12 67.242081) (width 0.4) (layer B.Cu) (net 7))
 (segment (start 73.66 60.015) (end 73.66 64.837919) (width 0.4) (layer B.Cu) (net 6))
 (segment (start 73.66 64.837919) (end 73.66 66.04) (width 0.4) (layer B.Cu) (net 6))
 (segment (start 77.16 56.515) (end 73.66 60.015) (width 0.4) (layer B.Cu) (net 6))
 (segment (start 78.31 56.515) (end 77.16 56.515) (width 0.4) (layer B.Cu) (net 6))
 (segment (start 73.66 66.04) (end 73.66 73.66) (width 0.4) (layer B.Cu) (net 6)))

